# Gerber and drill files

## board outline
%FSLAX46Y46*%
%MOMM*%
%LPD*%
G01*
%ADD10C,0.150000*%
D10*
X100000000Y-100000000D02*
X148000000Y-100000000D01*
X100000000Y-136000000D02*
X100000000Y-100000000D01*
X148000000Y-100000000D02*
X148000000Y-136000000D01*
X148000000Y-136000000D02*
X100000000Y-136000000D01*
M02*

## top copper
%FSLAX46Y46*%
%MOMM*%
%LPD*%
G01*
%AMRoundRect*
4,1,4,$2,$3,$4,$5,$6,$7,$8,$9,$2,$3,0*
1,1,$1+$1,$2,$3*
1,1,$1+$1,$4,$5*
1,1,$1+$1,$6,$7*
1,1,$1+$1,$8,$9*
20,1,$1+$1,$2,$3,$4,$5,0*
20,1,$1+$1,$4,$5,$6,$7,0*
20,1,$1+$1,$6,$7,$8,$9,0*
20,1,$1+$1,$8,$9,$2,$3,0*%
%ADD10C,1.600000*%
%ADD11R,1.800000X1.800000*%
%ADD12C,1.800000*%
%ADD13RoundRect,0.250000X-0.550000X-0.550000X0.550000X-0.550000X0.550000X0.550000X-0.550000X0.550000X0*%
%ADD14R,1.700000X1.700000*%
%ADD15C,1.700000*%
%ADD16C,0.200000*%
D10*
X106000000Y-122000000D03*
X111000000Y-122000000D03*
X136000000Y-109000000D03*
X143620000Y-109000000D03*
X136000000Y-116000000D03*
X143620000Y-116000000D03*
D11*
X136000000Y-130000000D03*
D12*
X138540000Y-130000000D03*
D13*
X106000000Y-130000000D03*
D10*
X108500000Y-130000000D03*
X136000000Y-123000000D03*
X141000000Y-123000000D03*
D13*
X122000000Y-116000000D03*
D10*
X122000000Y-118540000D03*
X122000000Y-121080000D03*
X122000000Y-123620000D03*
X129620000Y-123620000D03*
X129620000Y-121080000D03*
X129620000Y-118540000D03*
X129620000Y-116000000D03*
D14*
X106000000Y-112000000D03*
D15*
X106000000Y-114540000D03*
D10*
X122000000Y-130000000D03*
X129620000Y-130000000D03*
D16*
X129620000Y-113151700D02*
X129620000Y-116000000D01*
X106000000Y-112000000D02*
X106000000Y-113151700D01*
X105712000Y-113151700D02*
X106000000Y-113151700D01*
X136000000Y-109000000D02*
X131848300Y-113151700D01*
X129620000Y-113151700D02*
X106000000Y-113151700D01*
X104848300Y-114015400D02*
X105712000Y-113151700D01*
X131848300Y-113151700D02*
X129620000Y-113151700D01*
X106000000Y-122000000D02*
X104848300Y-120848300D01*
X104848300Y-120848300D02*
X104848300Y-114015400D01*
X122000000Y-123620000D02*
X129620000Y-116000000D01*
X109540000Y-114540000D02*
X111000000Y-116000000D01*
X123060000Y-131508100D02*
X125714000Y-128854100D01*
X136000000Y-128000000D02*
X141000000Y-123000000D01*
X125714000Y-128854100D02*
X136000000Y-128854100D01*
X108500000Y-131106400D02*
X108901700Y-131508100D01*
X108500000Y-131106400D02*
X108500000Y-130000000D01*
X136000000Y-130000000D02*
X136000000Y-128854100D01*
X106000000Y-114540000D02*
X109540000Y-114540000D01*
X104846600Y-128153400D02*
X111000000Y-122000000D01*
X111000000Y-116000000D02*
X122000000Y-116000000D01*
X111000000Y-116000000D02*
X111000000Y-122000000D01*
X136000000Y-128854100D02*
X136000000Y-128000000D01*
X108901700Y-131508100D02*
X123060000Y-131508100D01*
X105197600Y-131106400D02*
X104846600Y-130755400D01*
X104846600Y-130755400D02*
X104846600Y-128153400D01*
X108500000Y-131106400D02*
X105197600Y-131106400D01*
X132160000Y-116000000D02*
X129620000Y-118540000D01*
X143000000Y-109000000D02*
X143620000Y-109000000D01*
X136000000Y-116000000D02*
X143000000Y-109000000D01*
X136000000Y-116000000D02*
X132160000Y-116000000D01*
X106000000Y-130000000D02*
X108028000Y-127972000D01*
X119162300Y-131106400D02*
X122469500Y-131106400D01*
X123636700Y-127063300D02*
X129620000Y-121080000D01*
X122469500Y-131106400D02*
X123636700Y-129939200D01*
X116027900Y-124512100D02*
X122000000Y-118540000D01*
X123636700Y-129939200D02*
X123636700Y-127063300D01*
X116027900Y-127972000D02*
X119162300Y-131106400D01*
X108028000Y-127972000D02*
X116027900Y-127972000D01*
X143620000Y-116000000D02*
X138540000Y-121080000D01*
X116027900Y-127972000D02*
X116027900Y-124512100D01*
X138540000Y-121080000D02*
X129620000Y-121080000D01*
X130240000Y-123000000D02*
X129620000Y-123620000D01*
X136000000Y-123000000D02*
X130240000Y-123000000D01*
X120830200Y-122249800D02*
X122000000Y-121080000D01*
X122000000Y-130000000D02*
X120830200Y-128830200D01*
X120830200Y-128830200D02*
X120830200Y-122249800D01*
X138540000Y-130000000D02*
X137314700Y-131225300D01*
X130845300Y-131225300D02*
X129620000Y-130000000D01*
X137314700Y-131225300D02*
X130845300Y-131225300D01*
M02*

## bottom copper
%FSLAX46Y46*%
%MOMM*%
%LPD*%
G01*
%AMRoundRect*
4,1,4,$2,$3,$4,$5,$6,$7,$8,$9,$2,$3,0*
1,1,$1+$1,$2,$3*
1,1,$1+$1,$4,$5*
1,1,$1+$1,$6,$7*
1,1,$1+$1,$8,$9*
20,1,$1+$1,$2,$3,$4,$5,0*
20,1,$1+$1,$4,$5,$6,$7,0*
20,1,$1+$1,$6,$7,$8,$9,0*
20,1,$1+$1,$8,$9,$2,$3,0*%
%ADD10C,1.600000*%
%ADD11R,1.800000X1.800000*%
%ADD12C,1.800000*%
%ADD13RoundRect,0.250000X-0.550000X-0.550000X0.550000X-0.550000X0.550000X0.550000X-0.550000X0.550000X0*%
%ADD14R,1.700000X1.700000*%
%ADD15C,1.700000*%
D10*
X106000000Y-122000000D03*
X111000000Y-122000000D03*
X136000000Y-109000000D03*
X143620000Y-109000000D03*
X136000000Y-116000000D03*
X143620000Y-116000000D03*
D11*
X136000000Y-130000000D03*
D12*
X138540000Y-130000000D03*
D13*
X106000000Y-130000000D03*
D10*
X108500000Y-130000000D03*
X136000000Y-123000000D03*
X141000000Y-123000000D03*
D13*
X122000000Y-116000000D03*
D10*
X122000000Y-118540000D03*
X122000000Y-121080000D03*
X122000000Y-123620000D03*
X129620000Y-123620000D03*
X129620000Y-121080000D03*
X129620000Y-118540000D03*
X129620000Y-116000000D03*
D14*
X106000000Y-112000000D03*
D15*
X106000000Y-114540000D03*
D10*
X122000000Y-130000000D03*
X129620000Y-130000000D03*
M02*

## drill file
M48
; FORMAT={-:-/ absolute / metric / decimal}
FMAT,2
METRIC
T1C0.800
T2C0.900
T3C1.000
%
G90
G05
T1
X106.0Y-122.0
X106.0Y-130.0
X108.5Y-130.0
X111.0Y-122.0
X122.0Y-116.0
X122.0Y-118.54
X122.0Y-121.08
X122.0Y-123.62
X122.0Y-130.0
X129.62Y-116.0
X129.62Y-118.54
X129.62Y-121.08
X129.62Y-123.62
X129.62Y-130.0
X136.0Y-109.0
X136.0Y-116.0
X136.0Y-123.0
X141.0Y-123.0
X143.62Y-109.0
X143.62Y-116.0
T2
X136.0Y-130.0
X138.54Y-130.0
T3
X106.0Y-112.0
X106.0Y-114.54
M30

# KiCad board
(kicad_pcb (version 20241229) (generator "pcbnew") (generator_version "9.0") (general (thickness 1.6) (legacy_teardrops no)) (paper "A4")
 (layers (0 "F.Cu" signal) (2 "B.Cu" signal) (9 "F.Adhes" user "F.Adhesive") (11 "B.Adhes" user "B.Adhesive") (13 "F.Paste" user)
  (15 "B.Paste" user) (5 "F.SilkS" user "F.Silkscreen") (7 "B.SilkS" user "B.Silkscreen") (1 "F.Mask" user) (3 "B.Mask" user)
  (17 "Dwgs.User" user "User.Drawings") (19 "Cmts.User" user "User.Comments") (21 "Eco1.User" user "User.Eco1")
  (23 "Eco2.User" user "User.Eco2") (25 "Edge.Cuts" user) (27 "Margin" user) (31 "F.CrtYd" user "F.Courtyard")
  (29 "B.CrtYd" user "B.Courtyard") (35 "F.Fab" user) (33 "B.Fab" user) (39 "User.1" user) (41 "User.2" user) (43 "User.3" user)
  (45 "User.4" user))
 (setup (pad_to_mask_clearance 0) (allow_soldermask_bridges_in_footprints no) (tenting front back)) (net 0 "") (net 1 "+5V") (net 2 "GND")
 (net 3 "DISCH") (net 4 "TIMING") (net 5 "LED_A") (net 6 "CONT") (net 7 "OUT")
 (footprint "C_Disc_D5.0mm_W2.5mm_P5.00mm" (layer "F.Cu") (at 106 122)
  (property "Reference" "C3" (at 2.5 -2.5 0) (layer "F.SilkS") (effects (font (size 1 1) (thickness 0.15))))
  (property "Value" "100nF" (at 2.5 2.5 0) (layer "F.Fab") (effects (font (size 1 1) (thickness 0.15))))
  (pad "1" thru_hole circle (at 0 0) (size 1.6 1.6) (drill 0.8) (layers "*.Cu" "*.Mask") (remove_unused_layers no) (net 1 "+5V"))
  (pad "2" thru_hole circle (at 5 0) (size 1.6 1.6) (drill 0.8) (layers "*.Cu" "*.Mask") (remove_unused_layers no) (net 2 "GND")))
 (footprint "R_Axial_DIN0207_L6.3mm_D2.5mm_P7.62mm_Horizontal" (layer "F.Cu") (at 136 109)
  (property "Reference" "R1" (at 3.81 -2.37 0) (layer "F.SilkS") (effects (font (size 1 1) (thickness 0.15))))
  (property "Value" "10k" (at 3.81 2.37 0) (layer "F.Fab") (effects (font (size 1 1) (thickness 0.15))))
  (pad "1" thru_hole circle (at 0 0) (size 1.6 1.6) (drill 0.8) (layers "*.Cu" "*.Mask") (remove_unused_layers no) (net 1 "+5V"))
  (pad "2" thru_hole circle (at 7.62 0) (size 1.6 1.6) (drill 0.8) (layers "*.Cu" "*.Mask") (remove_unused_layers no) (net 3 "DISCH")))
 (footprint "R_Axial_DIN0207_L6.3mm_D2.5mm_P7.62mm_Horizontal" (layer "F.Cu") (at 136 116)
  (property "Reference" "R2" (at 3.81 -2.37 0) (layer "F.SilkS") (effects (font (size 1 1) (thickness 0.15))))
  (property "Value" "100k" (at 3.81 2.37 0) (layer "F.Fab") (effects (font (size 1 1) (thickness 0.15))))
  (pad "1" thru_hole circle (at 0 0) (size 1.6 1.6) (drill 0.8) (layers "*.Cu" "*.Mask") (remove_unused_layers no) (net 3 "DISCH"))
  (pad "2" thru_hole circle (at 7.62 0) (size 1.6 1.6) (drill 0.8) (layers "*.Cu" "*.Mask") (remove_unused_layers no) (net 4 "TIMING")))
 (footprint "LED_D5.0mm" (layer "F.Cu") (at 136 130)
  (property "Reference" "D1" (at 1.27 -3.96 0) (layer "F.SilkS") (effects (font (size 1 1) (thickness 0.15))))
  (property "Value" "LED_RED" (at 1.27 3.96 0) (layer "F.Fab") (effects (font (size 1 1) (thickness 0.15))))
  (pad "1" thru_hole rect (at 0 0) (size 1.8 1.8) (drill 0.9) (layers "*.Cu" "*.Mask") (remove_unused_layers no) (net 2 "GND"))
  (pad "2" thru_hole circle (at 2.54 0) (size 1.8 1.8) (drill 0.9) (layers "*.Cu" "*.Mask") (remove_unused_layers no) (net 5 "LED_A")))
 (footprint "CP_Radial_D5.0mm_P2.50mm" (layer "F.Cu") (at 106 130)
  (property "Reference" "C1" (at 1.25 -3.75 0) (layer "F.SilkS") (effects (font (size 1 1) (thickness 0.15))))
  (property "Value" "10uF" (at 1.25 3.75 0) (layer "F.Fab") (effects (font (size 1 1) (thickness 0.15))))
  (pad "1" thru_hole roundrect (at 0 0) (size 1.6 1.6) (drill 0.8) (layers "*.Cu" "*.Mask") (remove_unused_layers no)
   (roundrect_rratio 0.15625) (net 4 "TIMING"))
  (pad "2" thru_hole circle (at 2.5 0) (size 1.6 1.6) (drill 0.8) (layers "*.Cu" "*.Mask") (remove_unused_layers no) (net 2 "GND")))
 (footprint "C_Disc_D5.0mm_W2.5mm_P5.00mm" (layer "F.Cu") (at 136 123)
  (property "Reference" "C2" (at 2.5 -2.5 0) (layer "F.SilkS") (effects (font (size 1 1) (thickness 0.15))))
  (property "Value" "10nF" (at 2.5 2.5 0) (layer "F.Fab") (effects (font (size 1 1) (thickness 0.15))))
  (pad "1" thru_hole circle (at 0 0) (size 1.6 1.6) (drill 0.8) (layers "*.Cu" "*.Mask") (remove_unused_layers no) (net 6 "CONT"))
  (pad "2" thru_hole circle (at 5 0) (size 1.6 1.6) (drill 0.8) (layers "*.Cu" "*.Mask") (remove_unused_layers no) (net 2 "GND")))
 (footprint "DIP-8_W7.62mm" (layer "F.Cu") (at 122 116)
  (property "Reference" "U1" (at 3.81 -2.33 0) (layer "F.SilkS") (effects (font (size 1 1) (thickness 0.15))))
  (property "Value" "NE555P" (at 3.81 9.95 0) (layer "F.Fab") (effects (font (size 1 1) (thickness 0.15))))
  (pad "1" thru_hole roundrect (at 0 0) (size 1.6 1.6) (drill 0.8) (layers "*.Cu" "*.Mask") (remove_unused_layers no)
   (roundrect_rratio 0.15625) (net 2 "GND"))
  (pad "2" thru_hole circle (at 0 2.54) (size 1.6 1.6) (drill 0.8) (layers "*.Cu" "*.Mask") (remove_unused_layers no) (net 4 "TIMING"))
  (pad "3" thru_hole circle (at 0 5.08) (size 1.6 1.6) (drill 0.8) (layers "*.Cu" "*.Mask") (remove_unused_layers no) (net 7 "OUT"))
  (pad "4" thru_hole circle (at 0 7.62) (size 1.6 1.6) (drill 0.8) (layers "*.Cu" "*.Mask") (remove_unused_layers no) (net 1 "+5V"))
  (pad "5" thru_hole circle (at 7.62 7.62) (size 1.6 1.6) (drill 0.8) (layers "*.Cu" "*.Mask") (remove_unused_layers no) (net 6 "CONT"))
  (pad "6" thru_hole circle (at 7.62 5.08) (size 1.6 1.6) (drill 0.8) (layers "*.Cu" "*.Mask") (remove_unused_layers no) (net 4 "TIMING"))
  (pad "7" thru_hole circle (at 7.62 2.54) (size 1.6 1.6) (drill 0.8) (layers "*.Cu" "*.Mask") (remove_unused_layers no) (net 3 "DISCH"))
  (pad "8" thru_hole circle (at 7.62 0) (size 1.6 1.6) (drill 0.8) (layers "*.Cu" "*.Mask") (remove_unused_layers no) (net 1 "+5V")))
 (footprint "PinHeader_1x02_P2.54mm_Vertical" (layer "F.Cu") (at 106 112)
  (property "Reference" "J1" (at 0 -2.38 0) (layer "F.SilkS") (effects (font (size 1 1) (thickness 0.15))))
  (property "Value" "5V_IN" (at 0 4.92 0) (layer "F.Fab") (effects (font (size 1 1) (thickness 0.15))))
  (pad "1" thru_hole rect (at 0 0) (size 1.7 1.7) (drill 1) (layers "*.Cu" "*.Mask") (remove_unused_layers no) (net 1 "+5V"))
  (pad "2" thru_hole circle (at 0 2.54) (size 1.7 1.7) (drill 1) (layers "*.Cu" "*.Mask") (remove_unused_layers no) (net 2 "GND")))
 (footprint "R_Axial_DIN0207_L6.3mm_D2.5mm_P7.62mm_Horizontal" (layer "F.Cu") (at 122 130)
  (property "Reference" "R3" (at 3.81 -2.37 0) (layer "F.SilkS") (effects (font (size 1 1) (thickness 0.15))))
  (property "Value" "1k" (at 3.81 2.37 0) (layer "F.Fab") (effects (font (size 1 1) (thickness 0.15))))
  (pad "1" thru_hole circle (at 0 0) (size 1.6 1.6) (drill 0.8) (layers "*.Cu" "*.Mask") (remove_unused_layers no) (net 7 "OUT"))
  (pad "2" thru_hole circle (at 7.62 0) (size 1.6 1.6) (drill 0.8) (layers "*.Cu" "*.Mask") (remove_unused_layers no) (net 5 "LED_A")))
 (gr_line (start 100 100) (end 148 100) (stroke (width 0.15) (type default)) (layer "Edge.Cuts"))
 (gr_line (start 100 136) (end 100 100) (stroke (width 0.15) (type default)) (layer "Edge.Cuts"))
 (gr_line (start 148 100) (end 148 136) (stroke (width 0.15) (type default)) (layer "Edge.Cuts"))
 (gr_line (start 148 136) (end 100 136) (stroke (width 0.15) (type default)) (layer "Edge.Cuts"))
 (segment (start 129.62 113.1517) (end 129.62 116) (width 0.2) (layer "F.Cu") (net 1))
 (segment (start 106 112) (end 106 113.1517) (width 0.2) (layer "F.Cu") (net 1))
 (segment (start 105.712 113.1517) (end 106 113.1517) (width 0.2) (layer "F.Cu") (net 1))
 (segment (start 136 109) (end 131.8483 113.1517) (width 0.2) (layer "F.Cu") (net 1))
 (segment (start 129.62 113.1517) (end 106 113.1517) (width 0.2) (layer "F.Cu") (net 1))
 (segment (start 104.8483 114.0154) (end 105.712 113.1517) (width 0.2) (layer "F.Cu") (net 1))
 (segment (start 131.8483 113.1517) (end 129.62 113.1517) (width 0.2) (layer "F.Cu") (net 1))
 (segment (start 106 122) (end 104.8483 120.8483) (width 0.2) (layer "F.Cu") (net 1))
 (segment (start 104.8483 120.8483) (end 104.8483 114.0154) (width 0.2) (layer "F.Cu") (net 1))
 (segment (start 122 123.62) (end 129.62 116) (width 0.2) (layer "F.Cu") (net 1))
 (segment (start 109.54 114.54) (end 111 116) (width 0.2) (layer "F.Cu") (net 2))
 (segment (start 123.06 131.5081) (end 125.714 128.8541) (width 0.2) (layer "F.Cu") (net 2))
 (segment (start 136 128) (end 141 123) (width 0.2) (layer "F.Cu") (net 2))
 (segment (start 125.714 128.8541) (end 136 128.8541) (width 0.2) (layer "F.Cu") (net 2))
 (segment (start 108.5 131.1064) (end 108.9017 131.5081) (width 0.2) (layer "F.Cu") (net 2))
 (segment (start 108.5 131.1064) (end 108.5 130) (width 0.2) (layer "F.Cu") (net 2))
 (segment (start 136 130) (end 136 128.8541) (width 0.2) (layer "F.Cu") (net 2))
 (segment (start 106 114.54) (end 109.54 114.54) (width 0.2) (layer "F.Cu") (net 2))
 (segment (start 104.8466 128.1534) (end 111 122) (width 0.2) (layer "F.Cu") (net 2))
 (segment (start 111 116) (end 122 116) (width 0.2) (layer "F.Cu") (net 2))
 (segment (start 111 116) (end 111 122) (width 0.2) (layer "F.Cu") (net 2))
 (segment (start 136 128.8541) (end 136 128) (width 0.2) (layer "F.Cu") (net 2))
 (segment (start 108.9017 131.5081) (end 123.06 131.5081) (width 0.2) (layer "F.Cu") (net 2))
 (segment (start 105.1976 131.1064) (end 104.8466 130.7554) (width 0.2) (layer "F.Cu") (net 2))
 (segment (start 104.8466 130.7554) (end 104.8466 128.1534) (width 0.2) (layer "F.Cu") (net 2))
 (segment (start 108.5 131.1064) (end 105.1976 131.1064) (width 0.2) (layer "F.Cu") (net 2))
 (segment (start 132.16 116) (end 129.62 118.54) (width 0.2) (layer "F.Cu") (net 3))
 (segment (start 143 109) (end 143.62 109) (width 0.2) (layer "F.Cu") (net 3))
 (segment (start 136 116) (end 143 109) (width 0.2) (layer "F.Cu") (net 3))
 (segment (start 136 116) (end 132.16 116) (width 0.2) (layer "F.Cu") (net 3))
 (segment (start 106 130) (end 108.028 127.972) (width 0.2) (layer "F.Cu") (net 4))
 (segment (start 119.1623 131.1064) (end 122.4695 131.1064) (width 0.2) (layer "F.Cu") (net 4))
 (segment (start 123.6367 127.0633) (end 129.62 121.08) (width 0.2) (layer "F.Cu") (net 4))
 (segment (start 122.4695 131.1064) (end 123.6367 129.9392) (width 0.2) (layer "F.Cu") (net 4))
 (segment (start 116.0279 124.5121) (end 122 118.54) (width 0.2) (layer "F.Cu") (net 4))
 (segment (start 123.6367 129.9392) (end 123.6367 127.0633) (width 0.2) (layer "F.Cu") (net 4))
 (segment (start 116.0279 127.972) (end 119.1623 131.1064) (width 0.2) (layer "F.Cu") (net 4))
 (segment (start 108.028 127.972) (end 116.0279 127.972) (width 0.2) (layer "F.Cu") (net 4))
 (segment (start 143.62 116) (end 138.54 121.08) (width 0.2) (layer "F.Cu") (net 4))
 (segment (start 116.0279 127.972) (end 116.0279 124.5121) (width 0.2) (layer "F.Cu") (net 4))
 (segment (start 138.54 121.08) (end 129.62 121.08) (width 0.2) (layer "F.Cu") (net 4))
 (segment (start 130.24 123) (end 129.62 123.62) (width 0.2) (layer "F.Cu") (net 6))
 (segment (start 136 123) (end 130.24 123) (width 0.2) (layer "F.Cu") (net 6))
 (segment (start 120.8302 122.2498) (end 122 121.08) (width 0.2) (layer "F.Cu") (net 7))
 (segment (start 122 130) (end 120.8302 128.8302) (width 0.2) (layer "F.Cu") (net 7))
 (segment (start 120.8302 128.8302) (end 120.8302 122.2498) (width 0.2) (layer "F.Cu") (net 7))
 (segment (start 138.54 130) (end 137.3147 131.2253) (width 0.2) (layer "F.Cu") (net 5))
 (segment (start 130.8453 131.2253) (end 129.62 130) (width 0.2) (layer "F.Cu") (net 5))
 (segment (start 137.3147 131.2253) (end 130.8453 131.2253) (width 0.2) (layer "F.Cu") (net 5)))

